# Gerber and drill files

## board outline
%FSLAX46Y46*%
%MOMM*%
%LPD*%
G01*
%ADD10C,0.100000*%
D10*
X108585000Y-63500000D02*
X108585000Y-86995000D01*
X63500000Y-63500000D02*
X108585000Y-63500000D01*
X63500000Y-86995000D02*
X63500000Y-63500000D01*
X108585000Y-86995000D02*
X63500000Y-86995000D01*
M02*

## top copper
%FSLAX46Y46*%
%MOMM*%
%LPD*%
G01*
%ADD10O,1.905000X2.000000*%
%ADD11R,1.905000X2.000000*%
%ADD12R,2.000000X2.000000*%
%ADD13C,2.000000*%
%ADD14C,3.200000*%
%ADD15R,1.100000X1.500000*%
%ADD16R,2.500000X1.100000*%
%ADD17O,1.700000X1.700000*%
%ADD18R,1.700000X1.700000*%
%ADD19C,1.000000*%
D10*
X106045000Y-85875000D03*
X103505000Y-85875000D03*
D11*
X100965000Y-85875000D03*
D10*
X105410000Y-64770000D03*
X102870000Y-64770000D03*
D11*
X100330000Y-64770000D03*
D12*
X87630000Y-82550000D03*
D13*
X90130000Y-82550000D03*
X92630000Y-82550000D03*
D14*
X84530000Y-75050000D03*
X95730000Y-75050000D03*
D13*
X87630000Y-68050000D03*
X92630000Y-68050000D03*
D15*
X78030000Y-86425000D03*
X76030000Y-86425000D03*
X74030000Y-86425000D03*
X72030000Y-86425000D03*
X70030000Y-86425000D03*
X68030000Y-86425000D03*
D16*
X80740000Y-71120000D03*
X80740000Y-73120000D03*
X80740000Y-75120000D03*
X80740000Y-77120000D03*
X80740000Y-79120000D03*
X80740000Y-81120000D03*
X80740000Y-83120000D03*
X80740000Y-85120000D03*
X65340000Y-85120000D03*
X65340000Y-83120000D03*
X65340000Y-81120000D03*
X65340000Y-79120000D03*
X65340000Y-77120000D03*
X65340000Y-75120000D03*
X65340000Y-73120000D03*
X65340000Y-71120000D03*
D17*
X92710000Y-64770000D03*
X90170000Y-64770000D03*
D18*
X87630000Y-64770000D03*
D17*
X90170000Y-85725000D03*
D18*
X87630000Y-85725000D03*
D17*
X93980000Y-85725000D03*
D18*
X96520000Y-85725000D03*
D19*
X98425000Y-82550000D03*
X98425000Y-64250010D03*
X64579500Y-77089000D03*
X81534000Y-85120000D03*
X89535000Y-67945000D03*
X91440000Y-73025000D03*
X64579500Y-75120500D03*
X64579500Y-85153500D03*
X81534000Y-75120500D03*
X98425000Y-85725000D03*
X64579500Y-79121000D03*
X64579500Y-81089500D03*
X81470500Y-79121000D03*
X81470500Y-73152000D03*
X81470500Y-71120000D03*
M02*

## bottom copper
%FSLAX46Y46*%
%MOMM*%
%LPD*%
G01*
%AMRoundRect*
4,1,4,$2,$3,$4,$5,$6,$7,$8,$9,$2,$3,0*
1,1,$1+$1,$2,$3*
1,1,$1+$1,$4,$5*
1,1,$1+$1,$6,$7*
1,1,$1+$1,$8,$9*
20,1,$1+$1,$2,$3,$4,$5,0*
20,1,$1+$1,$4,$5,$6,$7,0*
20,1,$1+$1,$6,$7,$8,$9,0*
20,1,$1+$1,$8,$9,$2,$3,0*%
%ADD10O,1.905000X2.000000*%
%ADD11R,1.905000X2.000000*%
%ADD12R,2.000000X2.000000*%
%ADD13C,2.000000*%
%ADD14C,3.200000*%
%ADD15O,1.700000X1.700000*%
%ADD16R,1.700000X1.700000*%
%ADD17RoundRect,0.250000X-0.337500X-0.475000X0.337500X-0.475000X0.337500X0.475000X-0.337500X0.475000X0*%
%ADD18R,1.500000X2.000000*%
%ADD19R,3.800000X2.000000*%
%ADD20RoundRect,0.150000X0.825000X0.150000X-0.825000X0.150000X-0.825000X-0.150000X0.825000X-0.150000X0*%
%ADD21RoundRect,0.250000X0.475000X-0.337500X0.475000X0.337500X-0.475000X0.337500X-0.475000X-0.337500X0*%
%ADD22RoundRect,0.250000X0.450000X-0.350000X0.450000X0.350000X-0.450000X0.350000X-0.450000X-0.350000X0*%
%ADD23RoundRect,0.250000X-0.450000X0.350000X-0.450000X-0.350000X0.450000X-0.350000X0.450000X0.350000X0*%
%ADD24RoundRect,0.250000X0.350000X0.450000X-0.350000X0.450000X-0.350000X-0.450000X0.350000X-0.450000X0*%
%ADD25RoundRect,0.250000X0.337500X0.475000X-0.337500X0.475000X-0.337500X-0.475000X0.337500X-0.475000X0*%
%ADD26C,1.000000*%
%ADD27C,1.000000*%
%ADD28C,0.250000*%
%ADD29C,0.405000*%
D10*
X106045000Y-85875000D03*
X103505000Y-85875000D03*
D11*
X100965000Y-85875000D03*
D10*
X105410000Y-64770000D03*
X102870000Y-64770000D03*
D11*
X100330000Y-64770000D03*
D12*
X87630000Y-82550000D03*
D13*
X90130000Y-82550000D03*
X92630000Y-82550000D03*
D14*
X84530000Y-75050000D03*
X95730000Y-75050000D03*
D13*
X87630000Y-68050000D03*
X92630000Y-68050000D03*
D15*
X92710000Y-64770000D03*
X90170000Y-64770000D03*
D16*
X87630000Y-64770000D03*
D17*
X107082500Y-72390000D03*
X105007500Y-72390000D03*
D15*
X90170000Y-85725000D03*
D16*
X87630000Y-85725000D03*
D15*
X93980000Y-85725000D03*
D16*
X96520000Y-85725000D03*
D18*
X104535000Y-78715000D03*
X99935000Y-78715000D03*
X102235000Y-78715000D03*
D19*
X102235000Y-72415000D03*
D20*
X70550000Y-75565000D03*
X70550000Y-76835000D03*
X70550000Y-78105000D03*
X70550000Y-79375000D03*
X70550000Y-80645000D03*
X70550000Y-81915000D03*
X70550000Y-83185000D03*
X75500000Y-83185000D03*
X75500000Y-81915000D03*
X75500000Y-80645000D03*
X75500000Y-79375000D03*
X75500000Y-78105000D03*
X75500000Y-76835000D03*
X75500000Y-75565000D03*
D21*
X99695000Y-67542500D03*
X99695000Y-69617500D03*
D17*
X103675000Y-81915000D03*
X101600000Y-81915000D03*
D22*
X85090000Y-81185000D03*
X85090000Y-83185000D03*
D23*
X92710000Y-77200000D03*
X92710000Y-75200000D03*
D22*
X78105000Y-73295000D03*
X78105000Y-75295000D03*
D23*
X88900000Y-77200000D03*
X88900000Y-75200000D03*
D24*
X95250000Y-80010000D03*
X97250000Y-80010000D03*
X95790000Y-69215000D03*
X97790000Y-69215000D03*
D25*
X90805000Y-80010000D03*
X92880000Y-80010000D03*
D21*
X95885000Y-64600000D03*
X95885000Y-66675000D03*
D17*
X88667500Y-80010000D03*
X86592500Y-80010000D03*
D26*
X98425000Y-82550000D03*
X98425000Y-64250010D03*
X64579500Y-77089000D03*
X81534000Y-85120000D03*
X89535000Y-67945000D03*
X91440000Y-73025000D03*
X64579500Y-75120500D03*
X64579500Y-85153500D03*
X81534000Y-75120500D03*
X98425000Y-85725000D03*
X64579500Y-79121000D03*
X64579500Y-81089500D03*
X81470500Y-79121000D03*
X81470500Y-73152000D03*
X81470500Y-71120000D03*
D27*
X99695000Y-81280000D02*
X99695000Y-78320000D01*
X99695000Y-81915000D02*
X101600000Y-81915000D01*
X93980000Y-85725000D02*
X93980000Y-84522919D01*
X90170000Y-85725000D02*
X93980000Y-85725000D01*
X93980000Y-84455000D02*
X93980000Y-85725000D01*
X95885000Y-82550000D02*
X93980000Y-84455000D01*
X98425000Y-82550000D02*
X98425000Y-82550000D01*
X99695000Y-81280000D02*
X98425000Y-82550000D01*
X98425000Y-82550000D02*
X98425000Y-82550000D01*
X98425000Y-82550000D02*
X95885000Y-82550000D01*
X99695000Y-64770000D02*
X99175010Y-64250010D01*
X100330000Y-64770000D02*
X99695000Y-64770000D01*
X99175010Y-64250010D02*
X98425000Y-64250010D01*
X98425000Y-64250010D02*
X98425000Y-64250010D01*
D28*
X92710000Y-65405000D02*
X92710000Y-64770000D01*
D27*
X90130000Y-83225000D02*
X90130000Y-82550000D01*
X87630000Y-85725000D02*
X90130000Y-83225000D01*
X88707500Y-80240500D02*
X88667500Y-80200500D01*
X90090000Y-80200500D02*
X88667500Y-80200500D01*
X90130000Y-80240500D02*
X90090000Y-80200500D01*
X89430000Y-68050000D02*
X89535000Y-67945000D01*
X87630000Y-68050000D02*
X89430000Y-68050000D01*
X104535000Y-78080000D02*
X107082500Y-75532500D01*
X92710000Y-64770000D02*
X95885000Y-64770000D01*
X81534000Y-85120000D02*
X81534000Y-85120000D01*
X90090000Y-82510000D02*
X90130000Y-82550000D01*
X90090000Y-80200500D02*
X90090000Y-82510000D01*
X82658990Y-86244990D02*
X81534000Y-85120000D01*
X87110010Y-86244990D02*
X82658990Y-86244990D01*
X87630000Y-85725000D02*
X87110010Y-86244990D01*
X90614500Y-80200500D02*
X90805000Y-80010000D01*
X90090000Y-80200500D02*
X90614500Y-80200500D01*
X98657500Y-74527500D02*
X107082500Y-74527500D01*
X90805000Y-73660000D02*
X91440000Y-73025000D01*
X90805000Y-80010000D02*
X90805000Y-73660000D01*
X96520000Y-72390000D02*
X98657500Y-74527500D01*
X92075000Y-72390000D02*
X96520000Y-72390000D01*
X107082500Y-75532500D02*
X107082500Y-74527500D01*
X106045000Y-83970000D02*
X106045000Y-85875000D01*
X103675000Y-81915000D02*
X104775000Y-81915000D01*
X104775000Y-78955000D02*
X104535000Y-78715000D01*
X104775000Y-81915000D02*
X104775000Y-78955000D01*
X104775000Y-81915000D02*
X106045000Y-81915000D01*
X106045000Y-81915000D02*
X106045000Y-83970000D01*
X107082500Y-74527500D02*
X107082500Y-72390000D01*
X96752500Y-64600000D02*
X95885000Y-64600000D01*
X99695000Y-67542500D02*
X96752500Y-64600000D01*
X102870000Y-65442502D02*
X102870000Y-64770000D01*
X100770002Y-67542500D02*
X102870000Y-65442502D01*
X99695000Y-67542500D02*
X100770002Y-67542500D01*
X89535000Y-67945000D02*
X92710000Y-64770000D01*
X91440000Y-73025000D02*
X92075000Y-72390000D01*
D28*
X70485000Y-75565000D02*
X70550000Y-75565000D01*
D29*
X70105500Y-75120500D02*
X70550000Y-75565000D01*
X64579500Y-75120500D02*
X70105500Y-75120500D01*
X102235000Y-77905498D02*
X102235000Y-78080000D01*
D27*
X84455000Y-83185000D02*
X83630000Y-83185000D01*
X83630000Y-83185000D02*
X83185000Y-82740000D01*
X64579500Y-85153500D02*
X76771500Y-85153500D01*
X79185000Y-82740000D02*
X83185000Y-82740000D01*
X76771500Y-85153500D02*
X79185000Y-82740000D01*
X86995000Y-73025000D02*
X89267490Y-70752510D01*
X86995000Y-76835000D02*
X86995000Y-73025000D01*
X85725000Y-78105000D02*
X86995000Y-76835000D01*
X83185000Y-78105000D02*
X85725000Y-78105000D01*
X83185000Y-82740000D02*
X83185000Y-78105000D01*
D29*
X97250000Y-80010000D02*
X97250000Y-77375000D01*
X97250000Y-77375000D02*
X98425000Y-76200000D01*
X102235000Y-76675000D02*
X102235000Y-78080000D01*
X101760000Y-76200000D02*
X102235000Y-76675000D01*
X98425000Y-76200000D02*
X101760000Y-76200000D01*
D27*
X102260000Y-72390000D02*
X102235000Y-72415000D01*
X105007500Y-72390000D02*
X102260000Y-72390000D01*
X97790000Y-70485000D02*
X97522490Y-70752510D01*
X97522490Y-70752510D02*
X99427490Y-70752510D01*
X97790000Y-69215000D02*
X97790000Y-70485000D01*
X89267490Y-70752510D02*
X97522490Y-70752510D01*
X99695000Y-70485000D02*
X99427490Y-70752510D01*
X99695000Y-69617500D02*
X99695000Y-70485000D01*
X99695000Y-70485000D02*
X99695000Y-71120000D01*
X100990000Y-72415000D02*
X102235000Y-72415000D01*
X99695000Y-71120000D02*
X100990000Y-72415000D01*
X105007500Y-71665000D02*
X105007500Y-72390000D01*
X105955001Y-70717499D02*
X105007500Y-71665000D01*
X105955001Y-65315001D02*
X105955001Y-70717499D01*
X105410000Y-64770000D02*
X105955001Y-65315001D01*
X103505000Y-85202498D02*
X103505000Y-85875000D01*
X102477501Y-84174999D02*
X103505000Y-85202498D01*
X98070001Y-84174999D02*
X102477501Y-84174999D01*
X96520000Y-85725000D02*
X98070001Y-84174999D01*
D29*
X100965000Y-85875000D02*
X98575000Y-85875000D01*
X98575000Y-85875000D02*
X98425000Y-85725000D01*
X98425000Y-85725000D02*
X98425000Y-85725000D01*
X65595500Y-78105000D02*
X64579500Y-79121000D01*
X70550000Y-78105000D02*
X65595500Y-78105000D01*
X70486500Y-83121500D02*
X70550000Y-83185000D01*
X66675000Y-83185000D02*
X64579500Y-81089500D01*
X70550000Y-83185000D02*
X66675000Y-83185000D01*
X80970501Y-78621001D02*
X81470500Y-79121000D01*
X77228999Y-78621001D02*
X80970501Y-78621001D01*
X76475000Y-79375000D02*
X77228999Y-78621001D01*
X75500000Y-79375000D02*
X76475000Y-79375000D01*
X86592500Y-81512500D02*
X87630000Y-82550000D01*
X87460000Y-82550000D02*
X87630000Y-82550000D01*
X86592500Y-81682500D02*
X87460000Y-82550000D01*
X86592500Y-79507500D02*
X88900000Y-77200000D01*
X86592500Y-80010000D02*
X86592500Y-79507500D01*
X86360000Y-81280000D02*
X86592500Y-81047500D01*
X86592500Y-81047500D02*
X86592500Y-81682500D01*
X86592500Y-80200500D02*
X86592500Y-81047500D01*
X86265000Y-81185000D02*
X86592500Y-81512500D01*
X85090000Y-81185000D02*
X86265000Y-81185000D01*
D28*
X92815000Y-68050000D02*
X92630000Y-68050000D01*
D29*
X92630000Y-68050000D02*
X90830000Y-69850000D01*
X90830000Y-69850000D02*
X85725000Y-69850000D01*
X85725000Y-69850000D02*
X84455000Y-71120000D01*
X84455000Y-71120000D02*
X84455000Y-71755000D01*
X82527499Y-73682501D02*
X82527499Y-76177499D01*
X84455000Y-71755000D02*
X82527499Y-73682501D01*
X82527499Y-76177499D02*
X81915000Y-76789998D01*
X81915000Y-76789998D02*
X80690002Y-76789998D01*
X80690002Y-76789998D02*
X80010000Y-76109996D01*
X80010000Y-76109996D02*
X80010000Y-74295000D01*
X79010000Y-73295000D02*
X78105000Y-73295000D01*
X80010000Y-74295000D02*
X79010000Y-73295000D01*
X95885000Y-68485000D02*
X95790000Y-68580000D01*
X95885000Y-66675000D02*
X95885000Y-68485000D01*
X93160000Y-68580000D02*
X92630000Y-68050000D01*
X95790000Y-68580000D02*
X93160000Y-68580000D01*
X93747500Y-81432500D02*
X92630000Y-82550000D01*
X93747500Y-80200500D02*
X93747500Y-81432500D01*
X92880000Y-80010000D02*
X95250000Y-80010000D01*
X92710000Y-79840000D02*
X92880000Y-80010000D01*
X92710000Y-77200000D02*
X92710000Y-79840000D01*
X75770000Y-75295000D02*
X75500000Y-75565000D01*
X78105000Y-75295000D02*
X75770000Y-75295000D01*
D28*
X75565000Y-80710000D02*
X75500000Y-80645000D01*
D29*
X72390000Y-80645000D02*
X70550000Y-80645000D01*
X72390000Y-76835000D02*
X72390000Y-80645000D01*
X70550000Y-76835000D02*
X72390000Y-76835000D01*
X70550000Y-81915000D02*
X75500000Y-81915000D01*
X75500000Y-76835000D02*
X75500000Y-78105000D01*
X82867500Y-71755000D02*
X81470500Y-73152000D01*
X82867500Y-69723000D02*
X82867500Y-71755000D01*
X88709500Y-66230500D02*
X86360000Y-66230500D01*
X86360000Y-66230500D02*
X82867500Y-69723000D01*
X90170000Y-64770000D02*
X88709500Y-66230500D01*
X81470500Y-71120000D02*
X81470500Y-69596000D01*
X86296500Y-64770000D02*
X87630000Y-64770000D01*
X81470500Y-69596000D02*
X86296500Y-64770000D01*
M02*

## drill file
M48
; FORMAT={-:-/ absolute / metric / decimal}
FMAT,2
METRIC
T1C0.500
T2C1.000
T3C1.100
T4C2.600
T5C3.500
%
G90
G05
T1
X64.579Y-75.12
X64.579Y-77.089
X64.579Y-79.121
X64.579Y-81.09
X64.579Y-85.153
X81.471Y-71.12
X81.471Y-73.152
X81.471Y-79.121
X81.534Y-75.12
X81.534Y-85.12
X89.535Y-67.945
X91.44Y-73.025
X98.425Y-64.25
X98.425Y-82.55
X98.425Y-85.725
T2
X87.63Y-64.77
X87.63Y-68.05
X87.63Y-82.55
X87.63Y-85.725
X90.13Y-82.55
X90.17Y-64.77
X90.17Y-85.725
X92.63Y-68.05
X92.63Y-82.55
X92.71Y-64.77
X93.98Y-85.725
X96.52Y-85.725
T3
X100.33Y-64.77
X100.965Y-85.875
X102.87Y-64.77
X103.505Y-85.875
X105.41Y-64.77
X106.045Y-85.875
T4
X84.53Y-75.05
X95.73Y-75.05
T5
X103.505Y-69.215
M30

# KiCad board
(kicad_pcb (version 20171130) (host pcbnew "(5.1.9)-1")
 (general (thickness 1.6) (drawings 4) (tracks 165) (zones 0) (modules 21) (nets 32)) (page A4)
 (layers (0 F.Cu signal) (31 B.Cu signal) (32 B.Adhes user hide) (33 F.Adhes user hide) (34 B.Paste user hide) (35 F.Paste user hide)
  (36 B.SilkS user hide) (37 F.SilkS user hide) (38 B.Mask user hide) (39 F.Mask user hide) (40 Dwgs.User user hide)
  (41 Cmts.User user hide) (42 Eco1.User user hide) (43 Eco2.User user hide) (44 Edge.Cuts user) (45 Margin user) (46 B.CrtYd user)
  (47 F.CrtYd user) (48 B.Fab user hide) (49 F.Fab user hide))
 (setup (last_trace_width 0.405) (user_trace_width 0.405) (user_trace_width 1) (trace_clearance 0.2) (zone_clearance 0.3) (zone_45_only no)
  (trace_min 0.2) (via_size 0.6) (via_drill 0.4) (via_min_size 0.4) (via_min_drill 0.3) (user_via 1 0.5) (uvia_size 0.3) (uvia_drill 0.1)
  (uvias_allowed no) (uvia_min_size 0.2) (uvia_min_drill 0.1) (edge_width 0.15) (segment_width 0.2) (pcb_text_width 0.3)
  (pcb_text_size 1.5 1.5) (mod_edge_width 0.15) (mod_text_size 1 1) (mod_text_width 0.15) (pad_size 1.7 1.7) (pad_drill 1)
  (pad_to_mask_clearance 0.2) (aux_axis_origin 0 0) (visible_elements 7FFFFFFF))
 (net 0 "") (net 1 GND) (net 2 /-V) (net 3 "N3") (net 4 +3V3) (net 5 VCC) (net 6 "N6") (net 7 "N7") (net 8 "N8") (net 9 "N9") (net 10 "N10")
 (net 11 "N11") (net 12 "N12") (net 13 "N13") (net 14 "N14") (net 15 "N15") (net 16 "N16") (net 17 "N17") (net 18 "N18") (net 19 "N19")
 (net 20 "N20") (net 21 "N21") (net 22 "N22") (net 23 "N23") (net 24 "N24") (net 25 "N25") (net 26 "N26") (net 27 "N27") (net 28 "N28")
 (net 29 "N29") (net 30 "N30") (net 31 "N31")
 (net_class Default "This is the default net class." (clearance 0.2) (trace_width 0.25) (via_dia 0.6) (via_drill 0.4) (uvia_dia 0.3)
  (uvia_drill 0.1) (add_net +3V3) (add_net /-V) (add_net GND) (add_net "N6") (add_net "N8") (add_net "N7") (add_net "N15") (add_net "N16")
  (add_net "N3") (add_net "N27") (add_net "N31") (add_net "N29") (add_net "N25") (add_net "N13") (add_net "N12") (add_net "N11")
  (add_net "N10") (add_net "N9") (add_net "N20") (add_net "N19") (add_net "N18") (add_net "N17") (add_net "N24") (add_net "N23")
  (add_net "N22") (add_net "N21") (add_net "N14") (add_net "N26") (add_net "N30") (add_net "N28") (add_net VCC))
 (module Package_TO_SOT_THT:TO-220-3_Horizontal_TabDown (layer F.Cu) (at 100.965 85.875)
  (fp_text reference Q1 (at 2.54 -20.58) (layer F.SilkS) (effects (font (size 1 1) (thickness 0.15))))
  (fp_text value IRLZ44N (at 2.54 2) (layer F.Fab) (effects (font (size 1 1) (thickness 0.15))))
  (pad 3 thru_hole oval (at 5.08 0) (size 1.905 2) (drill 1.1) (layers *.Cu *.Mask) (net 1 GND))
  (pad 2 thru_hole oval (at 2.54 0) (size 1.905 2) (drill 1.1) (layers *.Cu *.Mask) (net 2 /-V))
  (pad 1 thru_hole rect (at 0 0) (size 1.905 2) (drill 1.1) (layers *.Cu *.Mask) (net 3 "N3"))
  (pad "" np_thru_hole oval (at 2.54 -16.66) (size 3.5 3.5) (drill 3.5) (layers *.Cu *.Mask)))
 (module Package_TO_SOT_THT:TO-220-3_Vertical (layer F.Cu) (at 100.33 64.77)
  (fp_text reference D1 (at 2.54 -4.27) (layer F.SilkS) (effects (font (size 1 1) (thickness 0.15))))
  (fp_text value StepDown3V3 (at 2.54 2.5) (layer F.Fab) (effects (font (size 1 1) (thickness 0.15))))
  (pad 3 thru_hole oval (at 5.08 0) (size 1.905 2) (drill 1.1) (layers *.Cu *.Mask) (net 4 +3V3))
  (pad 2 thru_hole oval (at 2.54 0) (size 1.905 2) (drill 1.1) (layers *.Cu *.Mask) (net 1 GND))
  (pad 1 thru_hole rect (at 0 0) (size 1.905 2) (drill 1.1) (layers *.Cu *.Mask) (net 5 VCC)))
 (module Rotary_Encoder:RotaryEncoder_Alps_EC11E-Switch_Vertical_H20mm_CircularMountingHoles (layer F.Cu) (at 87.63 82.55 90)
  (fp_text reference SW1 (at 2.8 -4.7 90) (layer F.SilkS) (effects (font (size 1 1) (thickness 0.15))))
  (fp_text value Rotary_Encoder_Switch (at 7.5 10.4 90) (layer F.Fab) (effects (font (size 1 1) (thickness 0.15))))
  (pad A thru_hole rect (at 0 0 90) (size 2 2) (drill 1) (layers *.Cu *.Mask) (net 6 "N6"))
  (pad C thru_hole circle (at 0 2.5 90) (size 2 2) (drill 1) (layers *.Cu *.Mask) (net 1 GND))
  (pad B thru_hole circle (at 0 5 90) (size 2 2) (drill 1) (layers *.Cu *.Mask) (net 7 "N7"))
  (pad MP thru_hole circle (at 7.5 -3.1 90) (size 3.2 3.2) (drill 2.6) (layers *.Cu *.Mask))
  (pad MP thru_hole circle (at 7.5 8.1 90) (size 3.2 3.2) (drill 2.6) (layers *.Cu *.Mask))
  (pad S2 thru_hole circle (at 14.5 0 90) (size 2 2) (drill 1) (layers *.Cu *.Mask) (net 1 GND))
  (pad S1 thru_hole circle (at 14.5 5 90) (size 2 2) (drill 1) (layers *.Cu *.Mask) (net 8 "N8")))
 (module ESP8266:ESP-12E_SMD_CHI (layer F.Cu) (at 66.04 71.12)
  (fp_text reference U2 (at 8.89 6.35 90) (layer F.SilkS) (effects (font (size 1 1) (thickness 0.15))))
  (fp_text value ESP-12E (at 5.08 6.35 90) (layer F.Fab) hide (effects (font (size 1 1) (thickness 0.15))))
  (pad 14 smd rect (at 11.99 14.605 90) (size 1.5 1.1) (drill (offset -0.7 0)) (layers F.Cu F.Paste F.Mask) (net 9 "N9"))
  (pad 13 smd rect (at 9.99 14.605 90) (size 1.5 1.1) (drill (offset -0.7 0)) (layers F.Cu F.Paste F.Mask) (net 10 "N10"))
  (pad 12 smd rect (at 7.99 14.605 90) (size 1.5 1.1) (drill (offset -0.7 0)) (layers F.Cu F.Paste F.Mask) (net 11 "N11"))
  (pad 11 smd rect (at 5.99 14.605 90) (size 1.5 1.1) (drill (offset -0.7 0)) (layers F.Cu F.Paste F.Mask) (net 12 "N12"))
  (pad 10 smd rect (at 3.99 14.605 90) (size 1.5 1.1) (drill (offset -0.7 0)) (layers F.Cu F.Paste F.Mask) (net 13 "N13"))
  (pad 9 smd rect (at 1.99 14.605 90) (size 1.5 1.1) (drill (offset -0.7 0)) (layers F.Cu F.Paste F.Mask) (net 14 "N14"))
  (pad 22 smd rect (at 14 0) (size 2.5 1.1) (drill (offset 0.7 0)) (layers F.Cu F.Paste F.Mask) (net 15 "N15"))
  (pad 21 smd rect (at 14 2) (size 2.5 1.1) (drill (offset 0.7 0)) (layers F.Cu F.Paste F.Mask) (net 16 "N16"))
  (pad 20 smd rect (at 14 4) (size 2.5 1.1) (drill (offset 0.7 0)) (layers F.Cu F.Paste F.Mask) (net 3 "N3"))
  (pad 19 smd rect (at 14 6) (size 2.5 1.1) (drill (offset 0.7 0)) (layers F.Cu F.Paste F.Mask) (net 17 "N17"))
  (pad 18 smd rect (at 14 8) (size 2.5 1.1) (drill (offset 0.7 0)) (layers F.Cu F.Paste F.Mask) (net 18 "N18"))
  (pad 17 smd rect (at 14 10) (size 2.5 1.1) (drill (offset 0.7 0)) (layers F.Cu F.Paste F.Mask) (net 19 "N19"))
  (pad 16 smd rect (at 14 12) (size 2.5 1.1) (drill (offset 0.7 0)) (layers F.Cu F.Paste F.Mask) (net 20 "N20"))
  (pad 15 smd rect (at 14 14) (size 2.5 1.1) (drill (offset 0.7 0)) (layers F.Cu F.Paste F.Mask) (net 1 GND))
  (pad 8 smd rect (at 0 14) (size 2.5 1.1) (drill (offset -0.7 0)) (layers F.Cu F.Paste F.Mask) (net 4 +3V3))
  (pad 7 smd rect (at 0 12) (size 2.5 1.1) (drill (offset -0.7 0)) (layers F.Cu F.Paste F.Mask) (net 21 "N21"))
  (pad 6 smd rect (at 0 10) (size 2.5 1.1) (drill (offset -0.7 0)) (layers F.Cu F.Paste F.Mask) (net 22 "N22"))
  (pad 5 smd rect (at 0 8) (size 2.5 1.1) (drill (offset -0.7 0)) (layers F.Cu F.Paste F.Mask) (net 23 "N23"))
  (pad 4 smd rect (at 0 6) (size 2.5 1.1) (drill (offset -0.7 0)) (layers F.Cu F.Paste F.Mask) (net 1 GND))
  (pad 3 smd rect (at 0 4) (size 2.5 1.1) (drill (offset -0.7 0)) (layers F.Cu F.Paste F.Mask) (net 4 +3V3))
  (pad 2 smd rect (at 0 2) (size 2.5 1.1) (drill (offset -0.7 0)) (layers F.Cu F.Paste F.Mask) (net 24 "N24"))
  (pad 1 smd rect (at 0 0) (size 2.5 1.1) (drill (offset -0.7 0)) (layers F.Cu F.Paste F.Mask) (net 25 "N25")))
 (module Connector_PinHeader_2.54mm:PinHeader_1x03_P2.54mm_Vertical (layer F.Cu) (at 87.63 64.77 90)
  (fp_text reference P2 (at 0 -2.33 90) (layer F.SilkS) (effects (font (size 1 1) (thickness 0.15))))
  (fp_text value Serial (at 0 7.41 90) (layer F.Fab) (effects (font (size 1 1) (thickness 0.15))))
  (pad 3 thru_hole oval (at 0 5.08 90) (size 1.7 1.7) (drill 1) (layers *.Cu *.Mask) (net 1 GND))
  (pad 2 thru_hole oval (at 0 2.54 90) (size 1.7 1.7) (drill 1) (layers *.Cu *.Mask) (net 16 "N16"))
  (pad 1 thru_hole rect (at 0 0 90) (size 1.7 1.7) (drill 1) (layers *.Cu *.Mask) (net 15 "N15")))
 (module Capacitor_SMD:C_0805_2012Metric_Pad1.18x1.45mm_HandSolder (layer B.Cu) (at 106.045 72.39)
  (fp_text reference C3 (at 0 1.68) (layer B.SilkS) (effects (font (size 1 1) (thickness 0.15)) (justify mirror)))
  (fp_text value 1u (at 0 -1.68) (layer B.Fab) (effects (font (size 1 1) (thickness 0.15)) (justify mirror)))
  (pad 2 smd roundrect (at 1.0375 0) (size 1.175 1.45) (layers B.Cu B.Paste B.Mask) (roundrect_rratio 0.212766) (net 1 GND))
  (pad 1 smd roundrect (at -1.0375 0) (size 1.175 1.45) (layers B.Cu B.Paste B.Mask) (roundrect_rratio 0.212766) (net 4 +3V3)))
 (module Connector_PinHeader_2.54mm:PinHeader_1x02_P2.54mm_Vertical (layer F.Cu) (at 87.63 85.725 90)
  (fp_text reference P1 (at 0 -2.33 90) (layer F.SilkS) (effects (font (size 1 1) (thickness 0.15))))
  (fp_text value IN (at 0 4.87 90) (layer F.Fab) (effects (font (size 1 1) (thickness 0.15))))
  (pad 2 thru_hole oval (at 0 2.54 90) (size 1.7 1.7) (drill 1) (layers *.Cu *.Mask) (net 5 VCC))
  (pad 1 thru_hole rect (at 0 0 90) (size 1.7 1.7) (drill 1) (layers *.Cu *.Mask) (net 1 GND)))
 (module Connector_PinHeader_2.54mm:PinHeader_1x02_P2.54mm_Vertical (layer F.Cu) (at 96.52 85.725 270)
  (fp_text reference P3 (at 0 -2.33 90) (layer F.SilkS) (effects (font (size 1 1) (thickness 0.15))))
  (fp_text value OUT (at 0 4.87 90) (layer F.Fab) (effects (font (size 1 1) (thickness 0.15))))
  (pad 2 thru_hole oval (at 0 2.54 270) (size 1.7 1.7) (drill 1) (layers *.Cu *.Mask) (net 5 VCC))
  (pad 1 thru_hole rect (at 0 0 270) (size 1.7 1.7) (drill 1) (layers *.Cu *.Mask) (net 2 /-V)))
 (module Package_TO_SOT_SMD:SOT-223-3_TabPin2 (layer B.Cu) (at 102.235 75.565 90)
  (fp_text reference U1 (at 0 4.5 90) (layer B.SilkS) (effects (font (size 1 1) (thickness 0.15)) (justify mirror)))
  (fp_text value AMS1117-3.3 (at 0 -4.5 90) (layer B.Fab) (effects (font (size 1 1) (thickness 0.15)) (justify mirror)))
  (pad 1 smd rect (at -3.15 2.3 90) (size 2 1.5) (layers B.Cu B.Paste B.Mask) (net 1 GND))
  (pad 3 smd rect (at -3.15 -2.3 90) (size 2 1.5) (layers B.Cu B.Paste B.Mask) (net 5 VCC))
  (pad 2 smd rect (at -3.15 0 90) (size 2 1.5) (layers B.Cu B.Paste B.Mask) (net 4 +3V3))
  (pad 2 smd rect (at 3.15 0 90) (size 2 3.8) (layers B.Cu B.Paste B.Mask) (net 4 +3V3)))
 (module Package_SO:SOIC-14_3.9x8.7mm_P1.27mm (layer B.Cu) (at 73.025 79.375 180)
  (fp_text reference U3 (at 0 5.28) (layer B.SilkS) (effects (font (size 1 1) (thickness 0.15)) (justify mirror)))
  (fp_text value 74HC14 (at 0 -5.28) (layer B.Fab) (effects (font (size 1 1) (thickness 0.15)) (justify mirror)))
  (pad 14 smd roundrect (at 2.475 3.81 180) (size 1.95 0.6) (layers B.Cu B.Paste B.Mask) (roundrect_rratio 0.25) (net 4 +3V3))
  (pad 13 smd roundrect (at 2.475 2.54 180) (size 1.95 0.6) (layers B.Cu B.Paste B.Mask) (roundrect_rratio 0.25) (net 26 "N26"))
  (pad 12 smd roundrect (at 2.475 1.27 180) (size 1.95 0.6) (layers B.Cu B.Paste B.Mask) (roundrect_rratio 0.25) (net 23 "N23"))
  (pad 11 smd roundrect (at 2.475 0 180) (size 1.95 0.6) (layers B.Cu B.Paste B.Mask) (roundrect_rratio 0.25) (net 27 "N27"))
  (pad 10 smd roundrect (at 2.475 -1.27 180) (size 1.95 0.6) (layers B.Cu B.Paste B.Mask) (roundrect_rratio 0.25) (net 26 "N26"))
  (pad 9 smd roundrect (at 2.475 -2.54 180) (size 1.95 0.6) (layers B.Cu B.Paste B.Mask) (roundrect_rratio 0.25) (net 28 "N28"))
  (pad 8 smd roundrect (at 2.475 -3.81 180) (size 1.95 0.6) (layers B.Cu B.Paste B.Mask) (roundrect_rratio 0.25) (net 22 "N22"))
  (pad 7 smd roundrect (at -2.475 -3.81 180) (size 1.95 0.6) (layers B.Cu B.Paste B.Mask) (roundrect_rratio 0.25) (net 1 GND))
  (pad 6 smd roundrect (at -2.475 -2.54 180) (size 1.95 0.6) (layers B.Cu B.Paste B.Mask) (roundrect_rratio 0.25) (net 28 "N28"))
  (pad 5 smd roundrect (at -2.475 -1.27 180) (size 1.95 0.6) (layers B.Cu B.Paste B.Mask) (roundrect_rratio 0.25) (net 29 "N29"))
  (pad 4 smd roundrect (at -2.475 0 180) (size 1.95 0.6) (layers B.Cu B.Paste B.Mask) (roundrect_rratio 0.25) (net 18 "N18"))
  (pad 3 smd roundrect (at -2.475 1.27 180) (size 1.95 0.6) (layers B.Cu B.Paste B.Mask) (roundrect_rratio 0.25) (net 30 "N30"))
  (pad 2 smd roundrect (at -2.475 2.54 180) (size 1.95 0.6) (layers B.Cu B.Paste B.Mask) (roundrect_rratio 0.25) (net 30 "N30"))
  (pad 1 smd roundrect (at -2.475 3.81 180) (size 1.95 0.6) (layers B.Cu B.Paste B.Mask) (roundrect_rratio 0.25) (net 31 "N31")))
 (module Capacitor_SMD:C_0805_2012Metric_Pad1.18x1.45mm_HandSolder (layer B.Cu) (at 99.695 68.58 90)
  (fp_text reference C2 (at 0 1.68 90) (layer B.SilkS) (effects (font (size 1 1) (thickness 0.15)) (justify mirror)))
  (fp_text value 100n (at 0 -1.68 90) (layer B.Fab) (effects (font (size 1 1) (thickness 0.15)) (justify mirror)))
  (pad 2 smd roundrect (at 1.0375 0 90) (size 1.175 1.45) (layers B.Cu B.Paste B.Mask) (roundrect_rratio 0.212766) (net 1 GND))
  (pad 1 smd roundrect (at -1.0375 0 90) (size 1.175 1.45) (layers B.Cu B.Paste B.Mask) (roundrect_rratio 0.212766) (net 4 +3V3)))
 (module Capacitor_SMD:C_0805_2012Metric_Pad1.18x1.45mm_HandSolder (layer B.Cu) (at 102.6375 81.915)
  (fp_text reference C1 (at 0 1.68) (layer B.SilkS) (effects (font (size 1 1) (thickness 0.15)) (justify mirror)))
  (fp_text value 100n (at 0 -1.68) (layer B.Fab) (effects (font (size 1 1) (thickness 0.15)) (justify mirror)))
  (pad 2 smd roundrect (at 1.0375 0) (size 1.175 1.45) (layers B.Cu B.Paste B.Mask) (roundrect_rratio 0.212766) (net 1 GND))
  (pad 1 smd roundrect (at -1.0375 0) (size 1.175 1.45) (layers B.Cu B.Paste B.Mask) (roundrect_rratio 0.212766) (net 5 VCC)))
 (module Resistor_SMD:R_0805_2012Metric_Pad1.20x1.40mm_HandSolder (layer B.Cu) (at 85.09 82.185 90)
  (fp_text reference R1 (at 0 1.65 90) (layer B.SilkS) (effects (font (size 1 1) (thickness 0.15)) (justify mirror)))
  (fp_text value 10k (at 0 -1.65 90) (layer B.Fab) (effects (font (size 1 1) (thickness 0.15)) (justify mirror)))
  (pad 2 smd roundrect (at 1 0 90) (size 1.2 1.4) (layers B.Cu B.Paste B.Mask) (roundrect_rratio 0.208333) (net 6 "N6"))
  (pad 1 smd roundrect (at -1 0 90) (size 1.2 1.4) (layers B.Cu B.Paste B.Mask) (roundrect_rratio 0.208333) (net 4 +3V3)))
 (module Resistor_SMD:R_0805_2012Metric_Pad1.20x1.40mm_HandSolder (layer B.Cu) (at 92.71 76.2 270)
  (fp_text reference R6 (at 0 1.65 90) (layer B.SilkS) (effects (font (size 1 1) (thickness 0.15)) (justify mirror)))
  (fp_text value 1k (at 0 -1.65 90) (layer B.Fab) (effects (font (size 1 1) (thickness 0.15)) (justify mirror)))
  (pad 2 smd roundrect (at 1 0 270) (size 1.2 1.4) (layers B.Cu B.Paste B.Mask) (roundrect_rratio 0.208333) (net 7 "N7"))
  (pad 1 smd roundrect (at -1 0 270) (size 1.2 1.4) (layers B.Cu B.Paste B.Mask) (roundrect_rratio 0.208333) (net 29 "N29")))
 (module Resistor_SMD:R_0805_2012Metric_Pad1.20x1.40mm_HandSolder (layer B.Cu) (at 78.105 74.295 90)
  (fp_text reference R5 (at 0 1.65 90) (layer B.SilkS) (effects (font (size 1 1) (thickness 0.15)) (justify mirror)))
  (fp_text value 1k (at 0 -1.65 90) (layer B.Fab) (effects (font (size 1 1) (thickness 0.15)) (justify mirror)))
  (pad 2 smd roundrect (at 1 0 90) (size 1.2 1.4) (layers B.Cu B.Paste B.Mask) (roundrect_rratio 0.208333) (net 8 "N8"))
  (pad 1 smd roundrect (at -1 0 90) (size 1.2 1.4) (layers B.Cu B.Paste B.Mask) (roundrect_rratio 0.208333) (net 31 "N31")))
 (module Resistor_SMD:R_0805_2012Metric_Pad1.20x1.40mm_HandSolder (layer B.Cu) (at 88.9 76.2 270)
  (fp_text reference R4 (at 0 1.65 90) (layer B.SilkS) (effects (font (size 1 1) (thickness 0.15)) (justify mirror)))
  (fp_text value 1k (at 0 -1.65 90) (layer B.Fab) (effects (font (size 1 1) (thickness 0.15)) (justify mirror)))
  (pad 2 smd roundrect (at 1 0 270) (size 1.2 1.4) (layers B.Cu B.Paste B.Mask) (roundrect_rratio 0.208333) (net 6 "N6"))
  (pad 1 smd roundrect (at -1 0 270) (size 1.2 1.4) (layers B.Cu B.Paste B.Mask) (roundrect_rratio 0.208333) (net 27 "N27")))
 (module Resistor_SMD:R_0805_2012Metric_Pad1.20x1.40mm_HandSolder (layer B.Cu) (at 96.25 80.01 180)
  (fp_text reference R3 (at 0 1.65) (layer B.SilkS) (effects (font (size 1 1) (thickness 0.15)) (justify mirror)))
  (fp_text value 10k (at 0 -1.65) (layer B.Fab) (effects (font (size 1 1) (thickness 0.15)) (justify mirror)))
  (pad 2 smd roundrect (at 1 0 180) (size 1.2 1.4) (layers B.Cu B.Paste B.Mask) (roundrect_rratio 0.208333) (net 7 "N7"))
  (pad 1 smd roundrect (at -1 0 180) (size 1.2 1.4) (layers B.Cu B.Paste B.Mask) (roundrect_rratio 0.208333) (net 4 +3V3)))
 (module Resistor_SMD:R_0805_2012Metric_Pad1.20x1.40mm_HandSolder (layer B.Cu) (at 96.79 69.215 180)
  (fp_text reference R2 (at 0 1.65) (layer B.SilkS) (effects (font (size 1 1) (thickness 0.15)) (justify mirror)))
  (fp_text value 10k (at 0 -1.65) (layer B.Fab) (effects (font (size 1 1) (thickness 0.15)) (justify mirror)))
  (pad 2 smd roundrect (at 1 0 180) (size 1.2 1.4) (layers B.Cu B.Paste B.Mask) (roundrect_rratio 0.208333) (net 8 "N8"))
  (pad 1 smd roundrect (at -1 0 180) (size 1.2 1.4) (layers B.Cu B.Paste B.Mask) (roundrect_rratio 0.208333) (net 4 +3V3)))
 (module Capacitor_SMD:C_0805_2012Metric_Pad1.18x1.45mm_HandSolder (layer B.Cu) (at 91.8425 80.01 180)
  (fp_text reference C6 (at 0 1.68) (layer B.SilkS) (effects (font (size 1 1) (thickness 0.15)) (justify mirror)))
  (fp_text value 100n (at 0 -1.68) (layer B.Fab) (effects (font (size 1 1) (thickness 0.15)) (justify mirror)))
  (pad 2 smd roundrect (at 1.0375 0 180) (size 1.175 1.45) (layers B.Cu B.Paste B.Mask) (roundrect_rratio 0.212766) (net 1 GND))
  (pad 1 smd roundrect (at -1.0375 0 180) (size 1.175 1.45) (layers B.Cu B.Paste B.Mask) (roundrect_rratio 0.212766) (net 7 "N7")))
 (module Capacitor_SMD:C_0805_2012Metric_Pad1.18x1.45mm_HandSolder (layer B.Cu) (at 95.885 65.6375 90)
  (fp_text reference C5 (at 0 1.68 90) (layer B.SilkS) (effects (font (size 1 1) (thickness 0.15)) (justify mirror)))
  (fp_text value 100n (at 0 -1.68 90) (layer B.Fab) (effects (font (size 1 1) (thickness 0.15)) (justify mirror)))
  (pad 2 smd roundrect (at 1.0375 0 90) (size 1.175 1.45) (layers B.Cu B.Paste B.Mask) (roundrect_rratio 0.212766) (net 1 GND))
  (pad 1 smd roundrect (at -1.0375 0 90) (size 1.175 1.45) (layers B.Cu B.Paste B.Mask) (roundrect_rratio 0.212766) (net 8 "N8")))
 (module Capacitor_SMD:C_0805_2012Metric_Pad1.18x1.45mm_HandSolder (layer B.Cu) (at 87.63 80.01)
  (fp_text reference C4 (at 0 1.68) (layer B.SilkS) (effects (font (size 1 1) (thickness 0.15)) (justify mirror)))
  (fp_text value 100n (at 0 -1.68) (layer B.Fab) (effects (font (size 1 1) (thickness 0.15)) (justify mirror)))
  (pad 2 smd roundrect (at 1.0375 0) (size 1.175 1.45) (layers B.Cu B.Paste B.Mask) (roundrect_rratio 0.212766) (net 1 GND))
  (pad 1 smd roundrect (at -1.0375 0) (size 1.175 1.45) (layers B.Cu B.Paste B.Mask) (roundrect_rratio 0.212766) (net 6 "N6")))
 (gr_line (start 108.585 63.5) (end 108.585 86.995) (layer Edge.Cuts) (width 0.1))
 (gr_line (start 63.5 63.5) (end 108.585 63.5) (layer Edge.Cuts) (width 0.1))
 (gr_line (start 63.5 86.995) (end 63.5 63.5) (layer Edge.Cuts) (width 0.1))
 (gr_line (start 108.585 86.995) (end 63.5 86.995) (layer Edge.Cuts) (width 0.1))
 (segment (start 99.695 81.28) (end 99.695 78.32) (width 1) (layer B.Cu) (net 5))
 (segment (start 99.695 81.915) (end 101.6 81.915) (width 1) (layer B.Cu) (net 5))
 (segment (start 93.98 85.725) (end 93.98 84.522919) (width 1) (layer B.Cu) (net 5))
 (segment (start 90.17 85.725) (end 93.98 85.725) (width 1) (layer B.Cu) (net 5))
 (segment (start 93.98 84.455) (end 93.98 85.725) (width 1) (layer B.Cu) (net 5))
 (segment (start 95.885 82.55) (end 93.98 84.455) (width 1) (layer B.Cu) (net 5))
 (segment (start 98.425 82.55) (end 98.425 82.55) (width 1) (layer B.Cu) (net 5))
 (segment (start 99.695 81.28) (end 98.425 82.55) (width 1) (layer B.Cu) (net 5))
 (segment (start 98.425 82.55) (end 98.425 82.55) (width 1) (layer B.Cu) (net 5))
 (segment (start 98.425 82.55) (end 95.885 82.55) (width 1) (layer B.Cu) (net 5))
 (via (at 98.425 82.55) (size 1) (drill 0.5) (layers F.Cu B.Cu) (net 5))
 (segment (start 99.695 64.77) (end 99.17501 64.25001) (width 1) (layer B.Cu) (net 5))
 (segment (start 100.33 64.77) (end 99.695 64.77) (width 1) (layer B.Cu) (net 5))
 (segment (start 99.17501 64.25001) (end 98.425 64.25001) (width 1) (layer B.Cu) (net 5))
 (segment (start 98.425 64.25001) (end 98.425 64.25001) (width 1) (layer B.Cu) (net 5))
 (via (at 98.425 64.25001) (size 1) (drill 0.5) (layers F.Cu B.Cu) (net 5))
 (via (at 64.5795 77.089) (size 1) (drill 0.5) (layers F.Cu B.Cu) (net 1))
 (segment (start 92.71 65.405) (end 92.71 64.77) (width 0.25) (layer B.Cu) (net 1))
 (segment (start 90.13 83.225) (end 90.13 82.55) (width 1) (layer B.Cu) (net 1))
 (segment (start 87.63 85.725) (end 90.13 83.225) (width 1) (layer B.Cu) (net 1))
 (segment (start 88.7075 80.2405) (end 88.6675 80.2005) (width 1) (layer B.Cu) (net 1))
 (segment (start 90.09 80.2005) (end 88.6675 80.2005) (width 1) (layer B.Cu) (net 1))
 (segment (start 90.13 80.2405) (end 90.09 80.2005) (width 1) (layer B.Cu) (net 1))
 (segment (start 89.43 68.05) (end 89.535 67.945) (width 1) (layer B.Cu) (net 1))
 (segment (start 87.63 68.05) (end 89.43 68.05) (width 1) (layer B.Cu) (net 1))
 (segment (start 104.535 78.08) (end 107.0825 75.5325) (width 1) (layer B.Cu) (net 1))
 (segment (start 92.71 64.77) (end 95.885 64.77) (width 1) (layer B.Cu) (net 1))
 (segment (start 81.534 85.12) (end 81.534 85.12) (width 1) (layer B.Cu) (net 1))
 (via (at 81.534 85.12) (size 1) (drill 0.5) (layers F.Cu B.Cu) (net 1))
 (segment (start 90.09 82.51) (end 90.13 82.55) (width 1) (layer B.Cu) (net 1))
 (segment (start 90.09 80.2005) (end 90.09 82.51) (width 1) (layer B.Cu) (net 1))
 (segment (start 82.65899 86.24499) (end 81.534 85.12) (width 1) (layer B.Cu) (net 1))
 (segment (start 87.11001 86.24499) (end 82.65899 86.24499) (width 1) (layer B.Cu) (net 1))
 (segment (start 87.63 85.725) (end 87.11001 86.24499) (width 1) (layer B.Cu) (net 1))
 (segment (start 90.6145 80.2005) (end 90.805 80.01) (width 1) (layer B.Cu) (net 1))
 (segment (start 90.09 80.2005) (end 90.6145 80.2005) (width 1) (layer B.Cu) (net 1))
 (segment (start 98.6575 74.5275) (end 107.0825 74.5275) (width 1) (layer B.Cu) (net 1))
 (segment (start 90.805 73.66) (end 91.44 73.025) (width 1) (layer B.Cu) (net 1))
 (segment (start 90.805 80.01) (end 90.805 73.66) (width 1) (layer B.Cu) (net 1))
 (segment (start 96.52 72.39) (end 98.6575 74.5275) (width 1) (layer B.Cu) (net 1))
 (segment (start 92.075 72.39) (end 96.52 72.39) (width 1) (layer B.Cu) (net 1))
 (segment (start 107.0825 75.5325) (end 107.0825 74.5275) (width 1) (layer B.Cu) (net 1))
 (segment (start 106.045 83.97) (end 106.045 85.875) (width 1) (layer B.Cu) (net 1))
 (segment (start 103.675 81.915) (end 104.775 81.915) (width 1) (layer B.Cu) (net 1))
 (segment (start 104.775 78.955) (end 104.535 78.715) (width 1) (layer B.Cu) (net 1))
 (segment (start 104.775 81.915) (end 104.775 78.955) (width 1) (layer B.Cu) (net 1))
 (segment (start 104.775 81.915) (end 106.045 81.915) (width 1) (layer B.Cu) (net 1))
 (segment (start 106.045 81.915) (end 106.045 83.97) (width 1) (layer B.Cu) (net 1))
 (segment (start 107.0825 74.5275) (end 107.0825 72.39) (width 1) (layer B.Cu) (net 1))
 (segment (start 96.7525 64.6) (end 95.885 64.6) (width 1) (layer B.Cu) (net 1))
 (segment (start 99.695 67.5425) (end 96.7525 64.6) (width 1) (layer B.Cu) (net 1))
 (segment (start 102.87 65.442502) (end 102.87 64.77) (width 1) (layer B.Cu) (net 1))
 (segment (start 100.770002 67.5425) (end 102.87 65.442502) (width 1) (layer B.Cu) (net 1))
 (segment (start 99.695 67.5425) (end 100.770002 67.5425) (width 1) (layer B.Cu) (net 1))
 (segment (start 89.535 67.945) (end 92.71 64.77) (width 1) (layer B.Cu) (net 1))
 (via (at 89.535 67.945) (size 1) (drill 0.5) (layers F.Cu B.Cu) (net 1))
 (segment (start 91.44 73.025) (end 92.075 72.39) (width 1) (layer B.Cu) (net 1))
 (via (at 91.44 73.025) (size 1) (drill 0.5) (layers F.Cu B.Cu) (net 1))
 (via (at 64.5795 75.1205) (size 1) (drill 0.5) (layers F.Cu B.Cu) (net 4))
 (via (at 64.5795 85.1535) (size 1) (drill 0.5) (layers F.Cu B.Cu) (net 4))
 (segment (start 70.485 75.565) (end 70.55 75.565) (width 0.25) (layer B.Cu) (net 4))
 (segment (start 70.1055 75.1205) (end 70.55 75.565) (width 0.405) (layer B.Cu) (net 4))
 (segment (start 64.5795 75.1205) (end 70.1055 75.1205) (width 0.405) (layer B.Cu) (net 4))
 (segment (start 102.235 77.905498) (end 102.235 78.08) (width 0.405) (layer B.Cu) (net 4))
 (segment (start 84.455 83.185) (end 83.63 83.185) (width 1) (layer B.Cu) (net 4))
 (segment (start 83.63 83.185) (end 83.185 82.74) (width 1) (layer B.Cu) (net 4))
 (segment (start 64.5795 85.1535) (end 76.7715 85.1535) (width 1) (layer B.Cu) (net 4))
 (segment (start 79.185 82.74) (end 83.185 82.74) (width 1) (layer B.Cu) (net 4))
 (segment (start 76.7715 85.1535) (end 79.185 82.74) (width 1) (layer B.Cu) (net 4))
 (segment (start 86.995 73.025) (end 89.26749 70.75251) (width 1) (layer B.Cu) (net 4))
 (segment (start 86.995 76.835) (end 86.995 73.025) (width 1) (layer B.Cu) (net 4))
 (segment (start 85.725 78.105) (end 86.995 76.835) (width 1) (layer B.Cu) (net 4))
 (segment (start 83.185 78.105) (end 85.725 78.105) (width 1) (layer B.Cu) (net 4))
 (segment (start 83.185 82.74) (end 83.185 78.105) (width 1) (layer B.Cu) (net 4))
 (segment (start 97.25 80.01) (end 97.25 77.375) (width 0.405) (layer B.Cu) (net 4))
 (segment (start 97.25 77.375) (end 98.425 76.2) (width 0.405) (layer B.Cu) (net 4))
 (segment (start 102.235 76.675) (end 102.235 78.08) (width 0.405) (layer B.Cu) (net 4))
 (segment (start 101.76 76.2) (end 102.235 76.675) (width 0.405) (layer B.Cu) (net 4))
 (segment (start 98.425 76.2) (end 101.76 76.2) (width 0.405) (layer B.Cu) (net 4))
 (segment (start 102.26 72.39) (end 102.235 72.415) (width 1) (layer B.Cu) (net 4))
 (segment (start 105.0075 72.39) (end 102.26 72.39) (width 1) (layer B.Cu) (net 4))
 (segment (start 97.79 70.485) (end 97.52249 70.75251) (width 1) (layer B.Cu) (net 4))
 (segment (start 97.52249 70.75251) (end 99.42749 70.75251) (width 1) (layer B.Cu) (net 4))
 (segment (start 97.79 69.215) (end 97.79 70.485) (width 1) (layer B.Cu) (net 4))
 (segment (start 89.26749 70.75251) (end 97.52249 70.75251) (width 1) (layer B.Cu) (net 4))
 (segment (start 99.695 70.485) (end 99.42749 70.75251) (width 1) (layer B.Cu) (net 4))
 (segment (start 99.695 69.6175) (end 99.695 70.485) (width 1) (layer B.Cu) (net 4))
 (segment (start 99.695 70.485) (end 99.695 71.12) (width 1) (layer B.Cu) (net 4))
 (segment (start 100.99 72.415) (end 102.235 72.415) (width 1) (layer B.Cu) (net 4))
 (segment (start 99.695 71.12) (end 100.99 72.415) (width 1) (layer B.Cu) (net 4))
 (segment (start 105.0075 71.665) (end 105.0075 72.39) (width 1) (layer B.Cu) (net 4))
 (segment (start 105.955001 70.717499) (end 105.0075 71.665) (width 1) (layer B.Cu) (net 4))
 (segment (start 105.955001 65.315001) (end 105.955001 70.717499) (width 1) (layer B.Cu) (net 4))
 (segment (start 105.41 64.77) (end 105.955001 65.315001) (width 1) (layer B.Cu) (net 4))
 (segment (start 103.505 85.202498) (end 103.505 85.875) (width 1) (layer B.Cu) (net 2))
 (segment (start 102.477501 84.174999) (end 103.505 85.202498) (width 1) (layer B.Cu) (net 2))
 (segment (start 98.070001 84.174999) (end 102.477501 84.174999) (width 1) (layer B.Cu) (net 2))
 (segment (start 96.52 85.725) (end 98.070001 84.174999) (width 1) (layer B.Cu) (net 2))
 (via (at 81.534 75.1205) (size 1) (drill 0.5) (layers F.Cu B.Cu) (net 3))
 (segment (start 100.965 85.875) (end 98.575 85.875) (width 0.405) (layer B.Cu) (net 3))
 (segment (start 98.575 85.875) (end 98.425 85.725) (width 0.405) (layer B.Cu) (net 3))
 (segment (start 98.425 85.725) (end 98.425 85.725) (width 0.405) (layer B.Cu) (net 3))
 (via (at 98.425 85.725) (size 1) (drill 0.5) (layers F.Cu B.Cu) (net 3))
 (via (at 64.5795 79.121) (size 1) (drill 0.5) (layers F.Cu B.Cu) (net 23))
 (segment (start 65.5955 78.105) (end 64.5795 79.121) (width 0.405) (layer B.Cu) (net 23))
 (segment (start 70.55 78.105) (end 65.5955 78.105) (width 0.405) (layer B.Cu) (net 23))
 (via (at 64.5795 81.0895) (size 1) (drill 0.5) (layers F.Cu B.Cu) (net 22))
 (segment (start 70.4865 83.1215) (end 70.55 83.185) (width 0.405) (layer B.Cu) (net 22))
 (segment (start 66.675 83.185) (end 64.5795 81.0895) (width 0.405) (layer B.Cu) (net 22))
 (segment (start 70.55 83.185) (end 66.675 83.185) (width 0.405) (layer B.Cu) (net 22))
 (via (at 81.4705 79.121) (size 1) (drill 0.5) (layers F.Cu B.Cu) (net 18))
 (segment (start 80.970501 78.621001) (end 81.4705 79.121) (width 0.405) (layer B.Cu) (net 18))
 (segment (start 77.228999 78.621001) (end 80.970501 78.621001) (width 0.405) (layer B.Cu) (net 18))
 (segment (start 76.475 79.375) (end 77.228999 78.621001) (width 0.405) (layer B.Cu) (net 18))
 (segment (start 75.5 79.375) (end 76.475 79.375) (width 0.405) (layer B.Cu) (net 18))
 (segment (start 86.5925 81.5125) (end 87.63 82.55) (width 0.405) (layer B.Cu) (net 6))
 (segment (start 87.46 82.55) (end 87.63 82.55) (width 0.405) (layer B.Cu) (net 6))
 (segment (start 86.5925 81.6825) (end 87.46 82.55) (width 0.405) (layer B.Cu) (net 6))
 (segment (start 86.5925 79.5075) (end 88.9 77.2) (width 0.405) (layer B.Cu) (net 6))
 (segment (start 86.5925 80.01) (end 86.5925 79.5075) (width 0.405) (layer B.Cu) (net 6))
 (segment (start 86.36 81.28) (end 86.5925 81.0475) (width 0.405) (layer B.Cu) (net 6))
 (segment (start 86.5925 81.0475) (end 86.5925 81.6825) (width 0.405) (layer B.Cu) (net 6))
 (segment (start 86.5925 80.2005) (end 86.5925 81.0475) (width 0.405) (layer B.Cu) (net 6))
 (segment (start 86.265 81.185) (end 86.5925 81.5125) (width 0.405) (layer B.Cu) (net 6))
 (segment (start 85.09 81.185) (end 86.265 81.185) (width 0.405) (layer B.Cu) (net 6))
 (segment (start 92.815 68.05) (end 92.63 68.05) (width 0.25) (layer B.Cu) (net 8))
 (segment (start 92.63 68.05) (end 90.83 69.85) (width 0.405) (layer B.Cu) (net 8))
 (segment (start 90.83 69.85) (end 85.725 69.85) (width 0.405) (layer B.Cu) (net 8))
 (segment (start 85.725 69.85) (end 84.455 71.12) (width 0.405) (layer B.Cu) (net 8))
 (segment (start 84.455 71.12) (end 84.455 71.755) (width 0.405) (layer B.Cu) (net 8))
 (segment (start 82.527499 73.682501) (end 82.527499 76.177499) (width 0.405) (layer B.Cu) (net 8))
 (segment (start 84.455 71.755) (end 82.527499 73.682501) (width 0.405) (layer B.Cu) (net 8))
 (segment (start 82.527499 76.177499) (end 81.915 76.789998) (width 0.405) (layer B.Cu) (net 8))
 (segment (start 81.915 76.789998) (end 80.690002 76.789998) (width 0.405) (layer B.Cu) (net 8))
 (segment (start 80.690002 76.789998) (end 80.01 76.109996) (width 0.405) (layer B.Cu) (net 8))
 (segment (start 80.01 76.109996) (end 80.01 74.295) (width 0.405) (layer B.Cu) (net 8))
 (segment (start 79.01 73.295) (end 78.105 73.295) (width 0.405) (layer B.Cu) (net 8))
 (segment (start 80.01 74.295) (end 79.01 73.295) (width 0.405) (layer B.Cu) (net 8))
 (segment (start 95.885 68.485) (end 95.79 68.58) (width 0.405) (layer B.Cu) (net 8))
 (segment (start 95.885 66.675) (end 95.885 68.485) (width 0.405) (layer B.Cu) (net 8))
 (segment (start 93.16 68.58) (end 92.63 68.05) (width 0.405) (layer B.Cu) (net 8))
 (segment (start 95.79 68.58) (end 93.16 68.58) (width 0.405) (layer B.Cu) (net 8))
 (segment (start 93.7475 81.4325) (end 92.63 82.55) (width 0.405) (layer B.Cu) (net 7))
 (segment (start 93.7475 80.2005) (end 93.7475 81.4325) (width 0.405) (layer B.Cu) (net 7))
 (segment (start 92.88 80.01) (end 95.25 80.01) (width 0.405) (layer B.Cu) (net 7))
 (segment (start 92.71 79.84) (end 92.88 80.01) (width 0.405) (layer B.Cu) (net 7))
 (segment (start 92.71 77.2) (end 92.71 79.84) (width 0.405) (layer B.Cu) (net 7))
 (segment (start 75.77 75.295) (end 75.5 75.565) (width 0.405) (layer B.Cu) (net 31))
 (segment (start 78.105 75.295) (end 75.77 75.295) (width 0.405) (layer B.Cu) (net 31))
 (segment (start 75.565 80.71) (end 75.5 80.645) (width 0.25) (layer B.Cu) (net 29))
 (segment (start 72.39 80.645) (end 70.55 80.645) (width 0.405) (layer B.Cu) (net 26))
 (segment (start 72.39 76.835) (end 72.39 80.645) (width 0.405) (layer B.Cu) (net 26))
 (segment (start 70.55 76.835) (end 72.39 76.835) (width 0.405) (layer B.Cu) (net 26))
 (segment (start 70.55 81.915) (end 75.5 81.915) (width 0.405) (layer B.Cu) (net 28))
 (segment (start 75.5 76.835) (end 75.5 78.105) (width 0.405) (layer B.Cu) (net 30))
 (via (at 81.4705 73.152) (size 1) (drill 0.5) (layers F.Cu B.Cu) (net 16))
 (segment (start 82.8675 71.755) (end 81.4705 73.152) (width 0.405) (layer B.Cu) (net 16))
 (segment (start 82.8675 69.723) (end 82.8675 71.755) (width 0.405) (layer B.Cu) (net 16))
 (segment (start 88.7095 66.2305) (end 86.36 66.2305) (width 0.405) (layer B.Cu) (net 16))
 (segment (start 86.36 66.2305) (end 82.8675 69.723) (width 0.405) (layer B.Cu) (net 16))
 (segment (start 90.17 64.77) (end 88.7095 66.2305) (width 0.405) (layer B.Cu) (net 16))
 (via (at 81.4705 71.12) (size 1) (drill 0.5) (layers F.Cu B.Cu) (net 15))
 (segment (start 81.4705 71.12) (end 81.4705 69.596) (width 0.405) (layer B.Cu) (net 15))
 (segment (start 86.2965 64.77) (end 87.63 64.77) (width 0.405) (layer B.Cu) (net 15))
 (segment (start 81.4705 69.596) (end 86.2965 64.77) (width 0.405) (layer B.Cu) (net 15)))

